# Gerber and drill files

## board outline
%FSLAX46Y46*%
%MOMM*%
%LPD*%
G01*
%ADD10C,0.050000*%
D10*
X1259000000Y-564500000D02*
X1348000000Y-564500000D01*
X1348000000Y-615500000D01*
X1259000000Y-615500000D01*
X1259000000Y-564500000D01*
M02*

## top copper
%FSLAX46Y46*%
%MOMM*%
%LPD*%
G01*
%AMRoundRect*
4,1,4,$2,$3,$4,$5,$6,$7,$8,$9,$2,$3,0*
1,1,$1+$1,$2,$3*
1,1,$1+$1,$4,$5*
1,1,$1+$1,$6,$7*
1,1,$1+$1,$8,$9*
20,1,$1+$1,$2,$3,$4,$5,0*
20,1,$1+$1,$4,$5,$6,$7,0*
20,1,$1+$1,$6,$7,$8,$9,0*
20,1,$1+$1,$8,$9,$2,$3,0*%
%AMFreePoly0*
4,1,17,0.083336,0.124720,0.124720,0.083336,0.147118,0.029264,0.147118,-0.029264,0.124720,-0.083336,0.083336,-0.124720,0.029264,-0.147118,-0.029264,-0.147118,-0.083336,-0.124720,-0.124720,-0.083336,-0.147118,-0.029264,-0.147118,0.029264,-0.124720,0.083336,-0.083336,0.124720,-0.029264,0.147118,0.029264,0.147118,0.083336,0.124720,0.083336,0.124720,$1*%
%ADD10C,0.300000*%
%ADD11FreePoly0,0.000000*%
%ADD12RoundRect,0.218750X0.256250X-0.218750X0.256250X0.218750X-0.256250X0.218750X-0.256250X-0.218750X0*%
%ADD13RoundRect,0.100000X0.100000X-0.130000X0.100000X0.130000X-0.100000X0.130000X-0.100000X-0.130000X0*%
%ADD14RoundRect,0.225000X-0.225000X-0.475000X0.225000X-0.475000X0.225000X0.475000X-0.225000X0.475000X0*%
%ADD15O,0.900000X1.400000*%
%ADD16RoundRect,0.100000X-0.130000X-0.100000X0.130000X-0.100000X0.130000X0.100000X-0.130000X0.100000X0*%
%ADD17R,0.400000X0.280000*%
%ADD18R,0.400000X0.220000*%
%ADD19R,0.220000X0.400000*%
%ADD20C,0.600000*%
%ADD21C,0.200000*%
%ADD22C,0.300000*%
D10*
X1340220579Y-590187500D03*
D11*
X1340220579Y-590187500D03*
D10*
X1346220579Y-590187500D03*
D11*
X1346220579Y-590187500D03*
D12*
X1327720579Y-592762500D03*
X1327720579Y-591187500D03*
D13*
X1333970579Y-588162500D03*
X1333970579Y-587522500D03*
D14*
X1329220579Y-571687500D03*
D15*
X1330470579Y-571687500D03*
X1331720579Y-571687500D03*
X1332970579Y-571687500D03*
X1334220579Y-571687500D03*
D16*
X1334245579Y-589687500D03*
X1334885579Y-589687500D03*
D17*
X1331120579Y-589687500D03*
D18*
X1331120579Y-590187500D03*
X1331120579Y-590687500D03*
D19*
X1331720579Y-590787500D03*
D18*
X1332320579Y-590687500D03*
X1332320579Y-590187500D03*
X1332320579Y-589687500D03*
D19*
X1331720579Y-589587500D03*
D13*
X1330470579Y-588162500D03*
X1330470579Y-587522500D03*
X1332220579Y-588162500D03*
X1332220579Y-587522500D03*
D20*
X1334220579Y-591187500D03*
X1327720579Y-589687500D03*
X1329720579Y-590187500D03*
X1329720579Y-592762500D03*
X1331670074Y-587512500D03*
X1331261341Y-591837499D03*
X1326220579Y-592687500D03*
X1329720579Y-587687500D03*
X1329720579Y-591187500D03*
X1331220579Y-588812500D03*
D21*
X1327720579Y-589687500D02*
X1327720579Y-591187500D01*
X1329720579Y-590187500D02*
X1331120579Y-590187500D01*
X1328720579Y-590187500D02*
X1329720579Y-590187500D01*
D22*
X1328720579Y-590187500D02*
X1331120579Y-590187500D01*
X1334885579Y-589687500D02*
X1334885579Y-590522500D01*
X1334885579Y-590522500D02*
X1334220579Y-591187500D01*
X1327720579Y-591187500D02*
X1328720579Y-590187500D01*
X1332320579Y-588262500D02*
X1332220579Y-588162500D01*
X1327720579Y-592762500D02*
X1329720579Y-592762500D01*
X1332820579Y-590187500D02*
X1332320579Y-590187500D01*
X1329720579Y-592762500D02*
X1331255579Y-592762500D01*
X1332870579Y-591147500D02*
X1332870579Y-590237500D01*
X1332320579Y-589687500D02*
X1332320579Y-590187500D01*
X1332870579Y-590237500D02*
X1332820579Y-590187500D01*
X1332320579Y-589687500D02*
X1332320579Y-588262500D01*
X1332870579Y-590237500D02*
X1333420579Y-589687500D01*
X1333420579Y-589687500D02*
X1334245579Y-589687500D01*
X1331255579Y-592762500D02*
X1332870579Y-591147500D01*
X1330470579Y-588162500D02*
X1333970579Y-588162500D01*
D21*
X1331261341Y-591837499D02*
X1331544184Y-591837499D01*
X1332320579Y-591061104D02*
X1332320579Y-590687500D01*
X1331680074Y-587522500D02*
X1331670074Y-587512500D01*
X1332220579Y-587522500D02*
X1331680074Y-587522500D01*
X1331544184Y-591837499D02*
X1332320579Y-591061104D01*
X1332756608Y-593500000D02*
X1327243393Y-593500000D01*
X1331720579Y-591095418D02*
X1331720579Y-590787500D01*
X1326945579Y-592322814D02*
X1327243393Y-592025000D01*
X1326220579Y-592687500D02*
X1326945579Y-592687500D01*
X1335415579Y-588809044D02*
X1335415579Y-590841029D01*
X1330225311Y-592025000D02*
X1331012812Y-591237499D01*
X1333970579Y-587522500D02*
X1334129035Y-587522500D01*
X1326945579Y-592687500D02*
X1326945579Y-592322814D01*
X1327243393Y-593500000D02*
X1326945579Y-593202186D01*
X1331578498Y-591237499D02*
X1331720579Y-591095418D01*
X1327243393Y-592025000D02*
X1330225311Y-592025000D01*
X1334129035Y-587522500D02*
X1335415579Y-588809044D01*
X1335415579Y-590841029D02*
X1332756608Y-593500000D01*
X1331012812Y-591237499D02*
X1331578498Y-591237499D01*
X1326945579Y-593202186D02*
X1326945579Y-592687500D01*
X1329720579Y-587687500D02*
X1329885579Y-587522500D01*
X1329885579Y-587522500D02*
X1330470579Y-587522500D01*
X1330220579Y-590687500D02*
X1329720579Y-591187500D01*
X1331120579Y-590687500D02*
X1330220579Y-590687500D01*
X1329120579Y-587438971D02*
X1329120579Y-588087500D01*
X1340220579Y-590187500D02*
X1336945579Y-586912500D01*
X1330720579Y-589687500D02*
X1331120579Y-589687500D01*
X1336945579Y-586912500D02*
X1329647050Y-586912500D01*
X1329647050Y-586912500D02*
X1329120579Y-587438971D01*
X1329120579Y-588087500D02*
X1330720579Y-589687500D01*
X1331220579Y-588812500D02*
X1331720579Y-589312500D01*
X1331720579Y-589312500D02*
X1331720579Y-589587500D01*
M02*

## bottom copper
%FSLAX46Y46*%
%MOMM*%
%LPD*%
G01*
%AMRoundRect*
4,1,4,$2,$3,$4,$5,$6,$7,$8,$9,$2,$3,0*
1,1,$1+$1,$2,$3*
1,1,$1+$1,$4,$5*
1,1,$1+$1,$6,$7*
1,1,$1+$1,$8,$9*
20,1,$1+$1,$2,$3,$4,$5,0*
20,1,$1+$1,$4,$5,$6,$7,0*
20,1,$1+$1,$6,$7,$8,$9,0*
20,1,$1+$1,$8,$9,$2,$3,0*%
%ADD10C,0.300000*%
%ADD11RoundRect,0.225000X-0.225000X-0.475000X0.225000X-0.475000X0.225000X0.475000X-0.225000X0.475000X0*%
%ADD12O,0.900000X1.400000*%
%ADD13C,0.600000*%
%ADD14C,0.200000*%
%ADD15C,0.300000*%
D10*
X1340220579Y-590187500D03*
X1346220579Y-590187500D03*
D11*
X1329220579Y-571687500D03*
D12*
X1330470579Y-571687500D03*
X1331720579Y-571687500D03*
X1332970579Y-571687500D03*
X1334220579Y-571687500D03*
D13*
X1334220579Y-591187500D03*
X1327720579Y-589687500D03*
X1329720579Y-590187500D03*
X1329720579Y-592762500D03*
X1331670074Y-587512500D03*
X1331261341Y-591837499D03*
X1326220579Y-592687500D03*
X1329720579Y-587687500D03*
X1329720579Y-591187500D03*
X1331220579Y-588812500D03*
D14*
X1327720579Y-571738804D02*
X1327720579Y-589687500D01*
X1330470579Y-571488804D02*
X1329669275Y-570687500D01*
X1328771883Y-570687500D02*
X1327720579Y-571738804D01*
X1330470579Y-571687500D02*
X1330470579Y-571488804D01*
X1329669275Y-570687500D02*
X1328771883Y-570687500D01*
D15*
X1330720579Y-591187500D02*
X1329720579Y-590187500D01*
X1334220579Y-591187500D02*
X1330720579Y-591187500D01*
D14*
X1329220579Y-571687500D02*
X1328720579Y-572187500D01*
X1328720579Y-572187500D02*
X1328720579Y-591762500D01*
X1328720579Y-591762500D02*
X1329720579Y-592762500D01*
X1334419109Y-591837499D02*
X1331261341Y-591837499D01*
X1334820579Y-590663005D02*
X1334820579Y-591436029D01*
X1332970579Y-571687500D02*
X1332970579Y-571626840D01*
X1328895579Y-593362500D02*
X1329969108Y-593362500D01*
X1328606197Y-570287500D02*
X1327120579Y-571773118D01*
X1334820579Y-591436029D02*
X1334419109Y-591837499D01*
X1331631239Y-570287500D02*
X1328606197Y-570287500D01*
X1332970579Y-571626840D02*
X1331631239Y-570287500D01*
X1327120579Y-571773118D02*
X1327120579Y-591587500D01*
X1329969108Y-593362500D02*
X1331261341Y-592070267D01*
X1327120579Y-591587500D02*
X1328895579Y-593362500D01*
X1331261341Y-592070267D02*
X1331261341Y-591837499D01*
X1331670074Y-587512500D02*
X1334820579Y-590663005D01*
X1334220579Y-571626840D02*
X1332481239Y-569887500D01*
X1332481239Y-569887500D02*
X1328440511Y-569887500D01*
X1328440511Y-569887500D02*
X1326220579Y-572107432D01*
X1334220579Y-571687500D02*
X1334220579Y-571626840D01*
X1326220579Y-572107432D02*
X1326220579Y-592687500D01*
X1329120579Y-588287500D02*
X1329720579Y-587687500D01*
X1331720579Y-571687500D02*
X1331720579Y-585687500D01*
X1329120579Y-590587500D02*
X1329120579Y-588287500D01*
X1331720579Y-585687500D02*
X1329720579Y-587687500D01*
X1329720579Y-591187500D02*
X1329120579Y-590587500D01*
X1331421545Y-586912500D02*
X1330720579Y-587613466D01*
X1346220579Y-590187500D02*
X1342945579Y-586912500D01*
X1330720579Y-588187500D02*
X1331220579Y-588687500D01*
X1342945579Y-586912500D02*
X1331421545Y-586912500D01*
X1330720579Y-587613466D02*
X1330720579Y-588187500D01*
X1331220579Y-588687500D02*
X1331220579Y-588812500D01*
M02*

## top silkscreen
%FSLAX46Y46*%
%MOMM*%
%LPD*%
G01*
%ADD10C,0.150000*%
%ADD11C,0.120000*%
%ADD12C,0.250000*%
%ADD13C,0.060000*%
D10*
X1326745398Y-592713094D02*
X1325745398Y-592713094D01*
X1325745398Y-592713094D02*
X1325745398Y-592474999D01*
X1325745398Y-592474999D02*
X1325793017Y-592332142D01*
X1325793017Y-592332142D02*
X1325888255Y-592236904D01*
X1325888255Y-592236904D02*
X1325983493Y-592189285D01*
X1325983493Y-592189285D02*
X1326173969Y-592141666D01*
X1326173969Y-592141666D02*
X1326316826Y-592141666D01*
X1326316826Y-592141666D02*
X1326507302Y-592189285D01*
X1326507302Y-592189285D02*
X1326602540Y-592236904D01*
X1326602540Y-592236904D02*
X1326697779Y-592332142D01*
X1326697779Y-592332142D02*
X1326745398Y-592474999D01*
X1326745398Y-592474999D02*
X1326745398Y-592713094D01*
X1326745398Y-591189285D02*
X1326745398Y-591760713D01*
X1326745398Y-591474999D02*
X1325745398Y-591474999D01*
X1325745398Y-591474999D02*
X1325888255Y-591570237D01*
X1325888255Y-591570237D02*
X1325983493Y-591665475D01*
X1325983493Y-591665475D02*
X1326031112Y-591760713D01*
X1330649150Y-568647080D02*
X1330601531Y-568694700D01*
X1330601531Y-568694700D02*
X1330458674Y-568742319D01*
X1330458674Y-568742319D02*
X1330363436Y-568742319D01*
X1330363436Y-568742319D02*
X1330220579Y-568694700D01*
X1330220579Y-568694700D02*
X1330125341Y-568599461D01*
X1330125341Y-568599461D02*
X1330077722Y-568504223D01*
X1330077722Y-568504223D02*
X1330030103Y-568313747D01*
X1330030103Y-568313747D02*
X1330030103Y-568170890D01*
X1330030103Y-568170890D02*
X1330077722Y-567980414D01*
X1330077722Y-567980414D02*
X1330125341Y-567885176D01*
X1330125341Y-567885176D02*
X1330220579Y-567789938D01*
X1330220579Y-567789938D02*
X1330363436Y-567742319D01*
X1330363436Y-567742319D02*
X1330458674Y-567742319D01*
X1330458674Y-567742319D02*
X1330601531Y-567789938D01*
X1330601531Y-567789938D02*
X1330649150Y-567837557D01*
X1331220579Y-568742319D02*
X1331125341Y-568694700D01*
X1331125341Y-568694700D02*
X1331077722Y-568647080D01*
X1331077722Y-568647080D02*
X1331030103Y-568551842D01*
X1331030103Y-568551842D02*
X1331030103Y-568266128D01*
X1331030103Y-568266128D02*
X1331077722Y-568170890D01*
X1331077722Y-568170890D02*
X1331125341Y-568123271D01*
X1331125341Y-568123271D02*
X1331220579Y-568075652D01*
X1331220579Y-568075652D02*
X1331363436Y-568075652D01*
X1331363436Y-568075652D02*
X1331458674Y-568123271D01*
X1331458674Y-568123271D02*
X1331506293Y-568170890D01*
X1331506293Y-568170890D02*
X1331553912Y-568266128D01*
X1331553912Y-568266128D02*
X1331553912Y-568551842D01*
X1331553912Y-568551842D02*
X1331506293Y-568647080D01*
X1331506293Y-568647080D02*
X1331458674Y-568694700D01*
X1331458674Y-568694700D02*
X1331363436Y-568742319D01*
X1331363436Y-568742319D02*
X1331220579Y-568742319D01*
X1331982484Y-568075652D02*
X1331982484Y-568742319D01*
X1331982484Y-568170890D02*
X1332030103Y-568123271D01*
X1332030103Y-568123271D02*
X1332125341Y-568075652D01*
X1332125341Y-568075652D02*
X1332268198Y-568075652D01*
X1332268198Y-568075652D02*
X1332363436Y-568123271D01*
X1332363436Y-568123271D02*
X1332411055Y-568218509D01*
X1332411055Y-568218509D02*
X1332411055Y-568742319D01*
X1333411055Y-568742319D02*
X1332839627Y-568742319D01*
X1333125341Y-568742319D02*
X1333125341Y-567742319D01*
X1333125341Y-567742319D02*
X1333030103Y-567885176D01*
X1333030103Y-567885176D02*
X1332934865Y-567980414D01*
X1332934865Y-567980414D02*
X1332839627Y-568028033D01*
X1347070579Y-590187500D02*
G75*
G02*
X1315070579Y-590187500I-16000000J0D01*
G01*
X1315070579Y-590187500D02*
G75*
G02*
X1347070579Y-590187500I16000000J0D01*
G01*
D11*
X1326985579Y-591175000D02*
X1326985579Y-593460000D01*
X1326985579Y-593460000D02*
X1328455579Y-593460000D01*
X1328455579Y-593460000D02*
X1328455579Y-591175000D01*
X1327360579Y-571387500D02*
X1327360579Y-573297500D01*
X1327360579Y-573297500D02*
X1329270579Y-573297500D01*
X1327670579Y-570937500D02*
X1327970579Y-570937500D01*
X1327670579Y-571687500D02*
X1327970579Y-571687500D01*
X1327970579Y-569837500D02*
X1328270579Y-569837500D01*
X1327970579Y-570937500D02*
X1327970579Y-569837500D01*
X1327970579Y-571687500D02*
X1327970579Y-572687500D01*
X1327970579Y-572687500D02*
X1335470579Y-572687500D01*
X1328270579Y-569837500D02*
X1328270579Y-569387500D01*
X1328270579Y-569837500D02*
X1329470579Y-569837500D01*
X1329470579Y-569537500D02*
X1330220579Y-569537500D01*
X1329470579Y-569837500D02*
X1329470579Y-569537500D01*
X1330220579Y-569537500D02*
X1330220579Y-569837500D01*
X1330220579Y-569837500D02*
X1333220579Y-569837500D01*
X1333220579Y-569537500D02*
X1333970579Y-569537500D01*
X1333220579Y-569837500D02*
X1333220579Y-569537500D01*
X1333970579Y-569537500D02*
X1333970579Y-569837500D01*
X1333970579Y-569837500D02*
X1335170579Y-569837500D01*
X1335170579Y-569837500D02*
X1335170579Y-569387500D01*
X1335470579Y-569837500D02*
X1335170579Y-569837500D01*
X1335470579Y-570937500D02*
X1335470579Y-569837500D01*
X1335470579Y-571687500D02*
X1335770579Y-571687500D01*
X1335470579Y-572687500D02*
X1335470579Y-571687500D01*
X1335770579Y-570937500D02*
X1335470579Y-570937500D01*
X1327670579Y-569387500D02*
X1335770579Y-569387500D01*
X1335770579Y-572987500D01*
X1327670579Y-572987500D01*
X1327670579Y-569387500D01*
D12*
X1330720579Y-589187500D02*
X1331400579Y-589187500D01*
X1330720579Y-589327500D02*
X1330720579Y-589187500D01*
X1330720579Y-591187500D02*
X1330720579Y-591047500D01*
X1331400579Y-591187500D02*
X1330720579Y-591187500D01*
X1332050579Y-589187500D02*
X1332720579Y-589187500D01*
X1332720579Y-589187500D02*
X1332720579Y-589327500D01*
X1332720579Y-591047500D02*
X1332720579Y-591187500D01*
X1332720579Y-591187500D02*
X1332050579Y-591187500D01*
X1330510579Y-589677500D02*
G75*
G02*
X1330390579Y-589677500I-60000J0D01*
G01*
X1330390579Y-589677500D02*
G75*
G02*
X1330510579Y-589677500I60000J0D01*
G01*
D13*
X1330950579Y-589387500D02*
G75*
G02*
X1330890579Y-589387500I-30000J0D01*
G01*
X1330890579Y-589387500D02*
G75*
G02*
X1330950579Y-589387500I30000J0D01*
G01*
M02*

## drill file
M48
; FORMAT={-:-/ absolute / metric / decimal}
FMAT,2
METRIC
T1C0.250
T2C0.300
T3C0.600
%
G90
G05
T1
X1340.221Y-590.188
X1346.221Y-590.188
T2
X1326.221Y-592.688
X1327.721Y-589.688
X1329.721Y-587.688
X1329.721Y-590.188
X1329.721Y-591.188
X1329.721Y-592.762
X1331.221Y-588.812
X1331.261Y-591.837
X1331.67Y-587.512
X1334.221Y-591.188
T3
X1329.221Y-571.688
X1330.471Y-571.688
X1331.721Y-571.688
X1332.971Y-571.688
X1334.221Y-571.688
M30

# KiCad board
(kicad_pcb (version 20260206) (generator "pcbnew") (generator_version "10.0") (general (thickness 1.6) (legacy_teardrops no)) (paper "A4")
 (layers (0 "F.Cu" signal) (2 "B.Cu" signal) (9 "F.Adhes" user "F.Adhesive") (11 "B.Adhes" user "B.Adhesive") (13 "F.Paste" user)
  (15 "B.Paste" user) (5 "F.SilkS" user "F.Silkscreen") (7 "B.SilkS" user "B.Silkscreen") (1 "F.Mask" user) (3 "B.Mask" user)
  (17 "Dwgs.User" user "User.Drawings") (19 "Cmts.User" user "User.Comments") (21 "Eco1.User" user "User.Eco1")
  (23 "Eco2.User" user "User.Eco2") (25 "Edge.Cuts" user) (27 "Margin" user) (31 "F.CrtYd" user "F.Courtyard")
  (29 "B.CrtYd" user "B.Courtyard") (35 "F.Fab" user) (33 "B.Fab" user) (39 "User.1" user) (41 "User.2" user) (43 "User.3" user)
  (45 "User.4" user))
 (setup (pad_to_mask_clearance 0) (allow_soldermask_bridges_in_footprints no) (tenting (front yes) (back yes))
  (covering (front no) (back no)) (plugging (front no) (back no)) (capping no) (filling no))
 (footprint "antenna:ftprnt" (layer "F.Cu") (at 1331.070579 575.1875)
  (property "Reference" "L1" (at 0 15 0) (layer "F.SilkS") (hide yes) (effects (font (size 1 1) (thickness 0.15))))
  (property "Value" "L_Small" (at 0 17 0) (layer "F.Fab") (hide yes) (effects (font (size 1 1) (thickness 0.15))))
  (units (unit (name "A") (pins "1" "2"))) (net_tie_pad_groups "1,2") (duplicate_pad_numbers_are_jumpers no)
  (fp_circle (center 0 15) (end 0 31) (stroke (width 0.15) (type solid)) (fill no) (layer "F.SilkS"))
  (pad "1" thru_hole circle (at 9.15 15) (size 0.3 0.3) (drill 0.25) (layers "*.Cu" "*.Mask") (remove_unused_layers no) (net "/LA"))
  (pad "1" smd custom (at 9.15 15) (size 0.3 0.3) (layers "F.Cu") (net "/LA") (zone_connect 0) (thermal_bridge_angle 90)
   (options (clearance outline) (anchor circle)) (primitives))
  (pad "2" thru_hole circle (at 15.15 15) (size 0.3 0.3) (drill 0.25) (layers "*.Cu" "*.Mask") (remove_unused_layers no) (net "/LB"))
  (pad "2" smd custom (at 15.15 15) (size 0.3 0.3) (layers "F.Cu") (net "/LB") (zone_connect 0) (thermal_bridge_angle 90)
   (options (clearance outline) (anchor circle)) (primitives)))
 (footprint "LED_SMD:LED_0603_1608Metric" (layer "F.Cu") (at 1327.720579 591.975 90)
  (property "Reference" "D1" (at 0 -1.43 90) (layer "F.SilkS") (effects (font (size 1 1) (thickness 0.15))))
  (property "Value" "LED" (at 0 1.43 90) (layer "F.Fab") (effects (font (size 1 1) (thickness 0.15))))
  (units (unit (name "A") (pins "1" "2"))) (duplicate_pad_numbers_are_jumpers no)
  (fp_line (start 0.8 -0.735) (end -1.485 -0.735) (stroke (width 0.12) (type solid)) (layer "F.SilkS"))
  (fp_line (start -1.485 -0.735) (end -1.485 0.735) (stroke (width 0.12) (type solid)) (layer "F.SilkS"))
  (fp_line (start -1.485 0.735) (end 0.8 0.735) (stroke (width 0.12) (type solid)) (layer "F.SilkS"))
  (pad "1" smd roundrect (at -0.7875 0 90) (size 0.875 0.95) (layers "F.Cu" "F.Mask" "F.Paste") (roundrect_rratio 0.25) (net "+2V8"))
  (pad "2" smd roundrect (at 0.7875 0 90) (size 0.875 0.95) (layers "F.Cu" "F.Mask" "F.Paste") (roundrect_rratio 0.25) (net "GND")))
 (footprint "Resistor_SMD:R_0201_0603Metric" (layer "F.Cu") (at 1333.970579 587.8425 90)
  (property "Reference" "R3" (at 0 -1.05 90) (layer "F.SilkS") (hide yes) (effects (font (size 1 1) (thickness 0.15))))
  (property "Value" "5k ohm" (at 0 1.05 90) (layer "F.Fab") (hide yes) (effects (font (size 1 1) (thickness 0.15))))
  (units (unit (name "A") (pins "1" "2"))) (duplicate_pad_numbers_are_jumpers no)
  (pad "" smd roundrect (at -0.345 0 90) (size 0.318 0.36) (layers "F.Paste") (roundrect_rratio 0.25))
  (pad "" smd roundrect (at 0.345 0 90) (size 0.318 0.36) (layers "F.Paste") (roundrect_rratio 0.25))
  (pad "1" smd roundrect (at -0.32 0 90) (size 0.46 0.4) (layers "F.Cu" "F.Mask") (roundrect_rratio 0.25) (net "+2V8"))
  (pad "2" smd roundrect (at 0.32 0 90) (size 0.46 0.4) (layers "F.Cu" "F.Mask") (roundrect_rratio 0.25) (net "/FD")))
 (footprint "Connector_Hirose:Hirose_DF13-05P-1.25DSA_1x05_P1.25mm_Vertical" (layer "F.Cu") (at 1329.220579 571.6875)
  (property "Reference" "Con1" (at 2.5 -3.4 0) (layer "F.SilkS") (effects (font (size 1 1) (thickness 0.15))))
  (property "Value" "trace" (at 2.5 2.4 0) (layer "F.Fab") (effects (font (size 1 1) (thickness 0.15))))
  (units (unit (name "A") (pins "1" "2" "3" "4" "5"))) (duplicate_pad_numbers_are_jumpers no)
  (fp_line (start -1.86 -0.3) (end -1.86 1.61) (stroke (width 0.12) (type solid)) (layer "F.SilkS"))
  (fp_line (start -1.86 1.61) (end 0.05 1.61) (stroke (width 0.12) (type solid)) (layer "F.SilkS"))
  (fp_line (start -1.55 -0.75) (end -1.25 -0.75) (stroke (width 0.12) (type solid)) (layer "F.SilkS"))
  (fp_line (start -1.55 0) (end -1.25 0) (stroke (width 0.12) (type solid)) (layer "F.SilkS"))
  (fp_line (start -1.25 -1.85) (end -0.95 -1.85) (stroke (width 0.12) (type solid)) (layer "F.SilkS"))
  (fp_line (start -1.25 -0.75) (end -1.25 -1.85) (stroke (width 0.12) (type solid)) (layer "F.SilkS"))
  (fp_line (start -1.25 0) (end -1.25 1) (stroke (width 0.12) (type solid)) (layer "F.SilkS"))
  (fp_line (start -1.25 1) (end 6.25 1) (stroke (width 0.12) (type solid)) (layer "F.SilkS"))
  (fp_line (start -0.95 -1.85) (end -0.95 -2.3) (stroke (width 0.12) (type solid)) (layer "F.SilkS"))
  (fp_line (start -0.95 -1.85) (end 0.25 -1.85) (stroke (width 0.12) (type solid)) (layer "F.SilkS"))
  (fp_line (start 0.25 -2.15) (end 1 -2.15) (stroke (width 0.12) (type solid)) (layer "F.SilkS"))
  (fp_line (start 0.25 -1.85) (end 0.25 -2.15) (stroke (width 0.12) (type solid)) (layer "F.SilkS"))
  (fp_line (start 1 -2.15) (end 1 -1.85) (stroke (width 0.12) (type solid)) (layer "F.SilkS"))
  (fp_line (start 1 -1.85) (end 4 -1.85) (stroke (width 0.12) (type solid)) (layer "F.SilkS"))
  (fp_line (start 4 -2.15) (end 4.75 -2.15) (stroke (width 0.12) (type solid)) (layer "F.SilkS"))
  (fp_line (start 4 -1.85) (end 4 -2.15) (stroke (width 0.12) (type solid)) (layer "F.SilkS"))
  (fp_line (start 4.75 -2.15) (end 4.75 -1.85) (stroke (width 0.12) (type solid)) (layer "F.SilkS"))
  (fp_line (start 4.75 -1.85) (end 5.95 -1.85) (stroke (width 0.12) (type solid)) (layer "F.SilkS"))
  (fp_line (start 5.95 -1.85) (end 5.95 -2.3) (stroke (width 0.12) (type solid)) (layer "F.SilkS"))
  (fp_line (start 6.25 -1.85) (end 5.95 -1.85) (stroke (width 0.12) (type solid)) (layer "F.SilkS"))
  (fp_line (start 6.25 -0.75) (end 6.25 -1.85) (stroke (width 0.12) (type solid)) (layer "F.SilkS"))
  (fp_line (start 6.25 0) (end 6.55 0) (stroke (width 0.12) (type solid)) (layer "F.SilkS"))
  (fp_line (start 6.25 1) (end 6.25 0) (stroke (width 0.12) (type solid)) (layer "F.SilkS"))
  (fp_line (start 6.55 -0.75) (end 6.25 -0.75) (stroke (width 0.12) (type solid)) (layer "F.SilkS"))
  (fp_rect (start -1.55 -2.3) (end 6.55 1.3) (stroke (width 0.12) (type solid)) (fill no) (layer "F.SilkS"))
  (pad "1" thru_hole roundrect (at 0 0) (size 0.9 1.4) (drill 0.6) (layers "*.Cu" "*.Mask") (remove_unused_layers no)
   (roundrect_rratio 0.25) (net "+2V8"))
  (pad "2" thru_hole oval (at 1.25 0) (size 0.9 1.4) (drill 0.6) (layers "*.Cu" "*.Mask") (remove_unused_layers no) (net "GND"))
  (pad "3" thru_hole oval (at 2.5 0) (size 0.9 1.4) (drill 0.6) (layers "*.Cu" "*.Mask") (remove_unused_layers no) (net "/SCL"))
  (pad "4" thru_hole oval (at 3.75 0) (size 0.9 1.4) (drill 0.6) (layers "*.Cu" "*.Mask") (remove_unused_layers no) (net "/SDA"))
  (pad "5" thru_hole oval (at 5 0) (size 0.9 1.4) (drill 0.6) (layers "*.Cu" "*.Mask") (remove_unused_layers no) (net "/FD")))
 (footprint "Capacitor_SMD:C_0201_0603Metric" (layer "F.Cu") (at 1334.565579 589.6875)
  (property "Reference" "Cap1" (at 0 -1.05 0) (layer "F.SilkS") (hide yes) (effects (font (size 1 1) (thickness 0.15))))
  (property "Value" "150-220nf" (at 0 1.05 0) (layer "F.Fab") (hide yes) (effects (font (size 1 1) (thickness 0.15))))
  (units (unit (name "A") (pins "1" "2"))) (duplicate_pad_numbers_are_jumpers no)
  (pad "" smd roundrect (at -0.345 0) (size 0.318 0.36) (layers "F.Paste") (roundrect_rratio 0.25))
  (pad "" smd roundrect (at 0.345 0) (size 0.318 0.36) (layers "F.Paste") (roundrect_rratio 0.25))
  (pad "1" smd roundrect (at -0.32 0) (size 0.46 0.4) (layers "F.Cu" "F.Mask") (roundrect_rratio 0.25) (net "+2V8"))
  (pad "2" smd roundrect (at 0.32 0) (size 0.46 0.4) (layers "F.Cu" "F.Mask") (roundrect_rratio 0.25) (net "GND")))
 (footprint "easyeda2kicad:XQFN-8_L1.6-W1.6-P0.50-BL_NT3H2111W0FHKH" (layer "F.Cu") (at 1331.720579 590.1875)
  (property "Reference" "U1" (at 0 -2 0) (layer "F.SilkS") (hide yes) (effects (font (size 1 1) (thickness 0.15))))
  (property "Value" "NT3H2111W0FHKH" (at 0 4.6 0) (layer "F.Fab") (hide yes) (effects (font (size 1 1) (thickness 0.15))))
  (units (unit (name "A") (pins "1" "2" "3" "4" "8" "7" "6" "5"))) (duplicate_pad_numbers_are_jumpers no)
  (fp_line (start -1 -1) (end -0.32 -1) (stroke (width 0.25) (type solid)) (layer "F.SilkS"))
  (fp_line (start -1 -0.86) (end -1 -1) (stroke (width 0.25) (type solid)) (layer "F.SilkS"))
  (fp_line (start -1 1) (end -1 0.86) (stroke (width 0.25) (type solid)) (layer "F.SilkS"))
  (fp_line (start -0.32 1) (end -1 1) (stroke (width 0.25) (type solid)) (layer "F.SilkS"))
  (fp_line (start 0.33 -1) (end 1 -1) (stroke (width 0.25) (type solid)) (layer "F.SilkS"))
  (fp_line (start 1 -1) (end 1 -0.86) (stroke (width 0.25) (type solid)) (layer "F.SilkS"))
  (fp_line (start 1 0.86) (end 1 1) (stroke (width 0.25) (type solid)) (layer "F.SilkS"))
  (fp_line (start 1 1) (end 0.33 1) (stroke (width 0.25) (type solid)) (layer "F.SilkS"))
  (fp_circle (center -1.27 -0.51) (end -1.21 -0.51) (stroke (width 0.25) (type solid)) (fill no) (layer "F.SilkS"))
  (fp_circle (center -0.8 -0.8) (end -0.77 -0.8) (stroke (width 0.06) (type solid)) (fill no) (layer "F.SilkS"))
  (pad "1" smd rect (at -0.6 -0.5) (size 0.4 0.28) (layers "F.Cu" "F.Mask" "F.Paste") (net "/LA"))
  (pad "2" smd rect (at -0.6 0) (size 0.4 0.22) (layers "F.Cu" "F.Mask" "F.Paste") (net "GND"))
  (pad "3" smd rect (at -0.6 0.5) (size 0.4 0.22) (layers "F.Cu" "F.Mask" "F.Paste") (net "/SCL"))
  (pad "4" smd rect (at 0 0.6 90) (size 0.4 0.22) (layers "F.Cu" "F.Mask" "F.Paste") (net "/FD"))
  (pad "5" smd rect (at 0.6 0.5) (size 0.4 0.22) (layers "F.Cu" "F.Mask" "F.Paste") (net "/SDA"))
  (pad "6" smd rect (at 0.6 0) (size 0.4 0.22) (layers "F.Cu" "F.Mask" "F.Paste") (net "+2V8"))
  (pad "7" smd rect (at 0.6 -0.5) (size 0.4 0.22) (layers "F.Cu" "F.Mask" "F.Paste") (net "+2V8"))
  (pad "8" smd rect (at 0 -0.6 90) (size 0.4 0.22) (layers "F.Cu" "F.Mask" "F.Paste") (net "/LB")))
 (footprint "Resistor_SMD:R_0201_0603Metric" (layer "F.Cu") (at 1330.470579 587.8425 90)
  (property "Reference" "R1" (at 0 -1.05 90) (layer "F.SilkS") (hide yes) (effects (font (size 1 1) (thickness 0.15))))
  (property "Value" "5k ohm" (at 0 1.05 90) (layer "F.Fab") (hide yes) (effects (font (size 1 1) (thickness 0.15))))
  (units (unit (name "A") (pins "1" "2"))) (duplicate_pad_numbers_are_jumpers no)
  (pad "" smd roundrect (at -0.345 0 90) (size 0.318 0.36) (layers "F.Paste") (roundrect_rratio 0.25))
  (pad "" smd roundrect (at 0.345 0 90) (size 0.318 0.36) (layers "F.Paste") (roundrect_rratio 0.25))
  (pad "1" smd roundrect (at -0.32 0 90) (size 0.46 0.4) (layers "F.Cu" "F.Mask") (roundrect_rratio 0.25) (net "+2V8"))
  (pad "2" smd roundrect (at 0.32 0 90) (size 0.46 0.4) (layers "F.Cu" "F.Mask") (roundrect_rratio 0.25) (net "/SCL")))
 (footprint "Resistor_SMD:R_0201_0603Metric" (layer "F.Cu") (at 1332.220579 587.8425 90)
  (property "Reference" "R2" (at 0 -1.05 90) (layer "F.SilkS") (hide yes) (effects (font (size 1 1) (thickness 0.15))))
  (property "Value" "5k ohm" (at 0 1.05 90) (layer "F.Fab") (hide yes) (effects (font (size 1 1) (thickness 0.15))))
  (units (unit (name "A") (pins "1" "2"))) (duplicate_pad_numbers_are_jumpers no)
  (pad "" smd roundrect (at -0.345 0 90) (size 0.318 0.36) (layers "F.Paste") (roundrect_rratio 0.25))
  (pad "" smd roundrect (at 0.345 0 90) (size 0.318 0.36) (layers "F.Paste") (roundrect_rratio 0.25))
  (pad "1" smd roundrect (at -0.32 0 90) (size 0.46 0.4) (layers "F.Cu" "F.Mask") (roundrect_rratio 0.25) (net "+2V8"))
  (pad "2" smd roundrect (at 0.32 0 90) (size 0.46 0.4) (layers "F.Cu" "F.Mask") (roundrect_rratio 0.25) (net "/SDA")))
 (gr_rect (start 1259 564.5) (end 1348 615.5) (stroke (width 0.05) (type default)) (fill no) (layer "Edge.Cuts"))
 (segment (start 1327.720579 589.6875) (end 1327.720579 591.1875) (width 0.2) (layer "F.Cu") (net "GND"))
 (segment (start 1329.720579 590.1875) (end 1331.120579 590.1875) (width 0.2) (layer "F.Cu") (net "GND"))
 (segment (start 1328.720579 590.1875) (end 1329.720579 590.1875) (width 0.2) (layer "F.Cu") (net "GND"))
 (segment (start 1328.720579 590.1875) (end 1331.120579 590.1875) (width 0.3) (layer "F.Cu") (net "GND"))
 (segment (start 1334.885579 589.6875) (end 1334.885579 590.5225) (width 0.3) (layer "F.Cu") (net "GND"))
 (segment (start 1334.885579 590.5225) (end 1334.220579 591.1875) (width 0.3) (layer "F.Cu") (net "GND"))
 (segment (start 1327.720579 591.1875) (end 1328.720579 590.1875) (width 0.3) (layer "F.Cu") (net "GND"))
 (via (at 1334.220579 591.1875) (size 0.6) (drill 0.3) (layers "F.Cu" "B.Cu") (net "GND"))
 (via (at 1327.720579 589.6875) (size 0.6) (drill 0.3) (layers "F.Cu" "B.Cu") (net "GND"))
 (via (at 1329.720579 590.1875) (size 0.6) (drill 0.3) (layers "F.Cu" "B.Cu") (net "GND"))
 (segment (start 1327.720579 571.738804) (end 1327.720579 589.6875) (width 0.2) (layer "B.Cu") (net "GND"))
 (segment (start 1330.470579 571.488804) (end 1329.669275 570.6875) (width 0.2) (layer "B.Cu") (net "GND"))
 (segment (start 1328.771883 570.6875) (end 1327.720579 571.738804) (width 0.2) (layer "B.Cu") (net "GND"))
 (segment (start 1330.470579 571.6875) (end 1330.470579 571.488804) (width 0.2) (layer "B.Cu") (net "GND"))
 (segment (start 1329.669275 570.6875) (end 1328.771883 570.6875) (width 0.2) (layer "B.Cu") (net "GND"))
 (segment (start 1330.720579 591.1875) (end 1329.720579 590.1875) (width 0.3) (layer "B.Cu") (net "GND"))
 (segment (start 1334.220579 591.1875) (end 1330.720579 591.1875) (width 0.3) (layer "B.Cu") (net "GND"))
 (segment (start 1332.320579 588.2625) (end 1332.220579 588.1625) (width 0.3) (layer "F.Cu") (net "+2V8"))
 (segment (start 1327.720579 592.7625) (end 1329.720579 592.7625) (width 0.3) (layer "F.Cu") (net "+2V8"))
 (segment (start 1332.820579 590.1875) (end 1332.320579 590.1875) (width 0.3) (layer "F.Cu") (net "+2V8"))
 (segment (start 1329.720579 592.7625) (end 1331.255579 592.7625) (width 0.3) (layer "F.Cu") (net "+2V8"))
 (segment (start 1332.870579 591.1475) (end 1332.870579 590.2375) (width 0.3) (layer "F.Cu") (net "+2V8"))
 (segment (start 1332.320579 589.6875) (end 1332.320579 590.1875) (width 0.3) (layer "F.Cu") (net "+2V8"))
 (segment (start 1332.870579 590.2375) (end 1332.820579 590.1875) (width 0.3) (layer "F.Cu") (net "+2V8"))
 (segment (start 1332.320579 589.6875) (end 1332.320579 588.2625) (width 0.3) (layer "F.Cu") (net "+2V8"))
 (segment (start 1332.870579 590.2375) (end 1333.420579 589.6875) (width 0.3) (layer "F.Cu") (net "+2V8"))
 (segment (start 1333.420579 589.6875) (end 1334.245579 589.6875) (width 0.3) (layer "F.Cu") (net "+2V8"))
 (segment (start 1331.255579 592.7625) (end 1332.870579 591.1475) (width 0.3) (layer "F.Cu") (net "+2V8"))
 (segment (start 1330.470579 588.1625) (end 1333.970579 588.1625) (width 0.3) (layer "F.Cu") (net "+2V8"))
 (via (at 1329.720579 592.7625) (size 0.6) (drill 0.3) (layers "F.Cu" "B.Cu") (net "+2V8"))
 (segment (start 1329.220579 571.6875) (end 1328.720579 572.1875) (width 0.2) (layer "B.Cu") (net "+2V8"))
 (segment (start 1328.720579 572.1875) (end 1328.720579 591.7625) (width 0.2) (layer "B.Cu") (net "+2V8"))
 (segment (start 1328.720579 591.7625) (end 1329.720579 592.7625) (width 0.2) (layer "B.Cu") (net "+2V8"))
 (segment (start 1331.261341 591.837499) (end 1331.544184 591.837499) (width 0.2) (layer "F.Cu") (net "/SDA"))
 (segment (start 1332.320579 591.061104) (end 1332.320579 590.6875) (width 0.2) (layer "F.Cu") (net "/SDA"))
 (segment (start 1331.680074 587.5225) (end 1331.670074 587.5125) (width 0.2) (layer "F.Cu") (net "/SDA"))
 (segment (start 1332.220579 587.5225) (end 1331.680074 587.5225) (width 0.2) (layer "F.Cu") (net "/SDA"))
 (segment (start 1331.544184 591.837499) (end 1332.320579 591.061104) (width 0.2) (layer "F.Cu") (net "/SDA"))
 (via (at 1331.670074 587.5125) (size 0.6) (drill 0.3) (layers "F.Cu" "B.Cu") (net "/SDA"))
 (via (at 1331.261341 591.837499) (size 0.6) (drill 0.3) (layers "F.Cu" "B.Cu") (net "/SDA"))
 (segment (start 1334.419109 591.837499) (end 1331.261341 591.837499) (width 0.2) (layer "B.Cu") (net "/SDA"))
 (segment (start 1334.820579 590.663005) (end 1334.820579 591.436029) (width 0.2) (layer "B.Cu") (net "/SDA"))
 (segment (start 1332.970579 571.6875) (end 1332.970579 571.62684) (width 0.2) (layer "B.Cu") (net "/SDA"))
 (segment (start 1328.895579 593.3625) (end 1329.969108 593.3625) (width 0.2) (layer "B.Cu") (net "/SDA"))
 (segment (start 1328.606197 570.2875) (end 1327.120579 571.773118) (width 0.2) (layer "B.Cu") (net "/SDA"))
 (segment (start 1334.820579 591.436029) (end 1334.419109 591.837499) (width 0.2) (layer "B.Cu") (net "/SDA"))
 (segment (start 1331.631239 570.2875) (end 1328.606197 570.2875) (width 0.2) (layer "B.Cu") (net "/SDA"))
 (segment (start 1332.970579 571.62684) (end 1331.631239 570.2875) (width 0.2) (layer "B.Cu") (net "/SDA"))
 (segment (start 1327.120579 571.773118) (end 1327.120579 591.5875) (width 0.2) (layer "B.Cu") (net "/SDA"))
 (segment (start 1329.969108 593.3625) (end 1331.261341 592.070267) (width 0.2) (layer "B.Cu") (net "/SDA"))
 (segment (start 1327.120579 591.5875) (end 1328.895579 593.3625) (width 0.2) (layer "B.Cu") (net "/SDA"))
 (segment (start 1331.261341 592.070267) (end 1331.261341 591.837499) (width 0.2) (layer "B.Cu") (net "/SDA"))
 (segment (start 1331.670074 587.5125) (end 1334.820579 590.663005) (width 0.2) (layer "B.Cu") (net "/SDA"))
 (segment (start 1332.756608 593.5) (end 1327.243393 593.5) (width 0.2) (layer "F.Cu") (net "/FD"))
 (segment (start 1331.720579 591.095418) (end 1331.720579 590.7875) (width 0.2) (layer "F.Cu") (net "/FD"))
 (segment (start 1326.945579 592.322814) (end 1327.243393 592.025) (width 0.2) (layer "F.Cu") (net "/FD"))
 (segment (start 1326.220579 592.6875) (end 1326.945579 592.6875) (width 0.2) (layer "F.Cu") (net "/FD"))
 (segment (start 1335.415579 588.809044) (end 1335.415579 590.841029) (width 0.2) (layer "F.Cu") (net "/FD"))
 (segment (start 1330.225311 592.025) (end 1331.012812 591.237499) (width 0.2) (layer "F.Cu") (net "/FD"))
 (segment (start 1333.970579 587.5225) (end 1334.129035 587.5225) (width 0.2) (layer "F.Cu") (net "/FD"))
 (segment (start 1326.945579 592.6875) (end 1326.945579 592.322814) (width 0.2) (layer "F.Cu") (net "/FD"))
 (segment (start 1327.243393 593.5) (end 1326.945579 593.202186) (width 0.2) (layer "F.Cu") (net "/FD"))
 (segment (start 1331.578498 591.237499) (end 1331.720579 591.095418) (width 0.2) (layer "F.Cu") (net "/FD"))
 (segment (start 1327.243393 592.025) (end 1330.225311 592.025) (width 0.2) (layer "F.Cu") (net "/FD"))
 (segment (start 1334.129035 587.5225) (end 1335.415579 588.809044) (width 0.2) (layer "F.Cu") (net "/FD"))
 (segment (start 1335.415579 590.841029) (end 1332.756608 593.5) (width 0.2) (layer "F.Cu") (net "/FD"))
 (segment (start 1331.012812 591.237499) (end 1331.578498 591.237499) (width 0.2) (layer "F.Cu") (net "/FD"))
 (segment (start 1326.945579 593.202186) (end 1326.945579 592.6875) (width 0.2) (layer "F.Cu") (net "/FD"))
 (via (at 1326.220579 592.6875) (size 0.6) (drill 0.3) (layers "F.Cu" "B.Cu") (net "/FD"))
 (segment (start 1334.220579 571.62684) (end 1332.481239 569.8875) (width 0.2) (layer "B.Cu") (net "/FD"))
 (segment (start 1332.481239 569.8875) (end 1328.440511 569.8875) (width 0.2) (layer "B.Cu") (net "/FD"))
 (segment (start 1328.440511 569.8875) (end 1326.220579 572.107432) (width 0.2) (layer "B.Cu") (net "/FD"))
 (segment (start 1334.220579 571.6875) (end 1334.220579 571.62684) (width 0.2) (layer "B.Cu") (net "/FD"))
 (segment (start 1326.220579 572.107432) (end 1326.220579 592.6875) (width 0.2) (layer "B.Cu") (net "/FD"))
 (segment (start 1329.720579 587.6875) (end 1329.885579 587.5225) (width 0.2) (layer "F.Cu") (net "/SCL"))
 (segment (start 1329.885579 587.5225) (end 1330.470579 587.5225) (width 0.2) (layer "F.Cu") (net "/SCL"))
 (segment (start 1330.220579 590.6875) (end 1329.720579 591.1875) (width 0.2) (layer "F.Cu") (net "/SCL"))
 (segment (start 1331.120579 590.6875) (end 1330.220579 590.6875) (width 0.2) (layer "F.Cu") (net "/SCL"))
 (via (at 1329.720579 587.6875) (size 0.6) (drill 0.3) (layers "F.Cu" "B.Cu") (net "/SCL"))
 (via (at 1329.720579 591.1875) (size 0.6) (drill 0.3) (layers "F.Cu" "B.Cu") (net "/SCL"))
 (segment (start 1329.120579 588.2875) (end 1329.720579 587.6875) (width 0.2) (layer "B.Cu") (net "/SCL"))
 (segment (start 1331.720579 571.6875) (end 1331.720579 585.6875) (width 0.2) (layer "B.Cu") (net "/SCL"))
 (segment (start 1329.120579 590.5875) (end 1329.120579 588.2875) (width 0.2) (layer "B.Cu") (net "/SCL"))
 (segment (start 1331.720579 585.6875) (end 1329.720579 587.6875) (width 0.2) (layer "B.Cu") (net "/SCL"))
 (segment (start 1329.720579 591.1875) (end 1329.120579 590.5875) (width 0.2) (layer "B.Cu") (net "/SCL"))
 (segment (start 1329.120579 587.438971) (end 1329.120579 588.0875) (width 0.2) (layer "F.Cu") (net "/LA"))
 (segment (start 1340.220579 590.1875) (end 1336.945579 586.9125) (width 0.2) (layer "F.Cu") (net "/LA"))
 (segment (start 1330.720579 589.6875) (end 1331.120579 589.6875) (width 0.2) (layer "F.Cu") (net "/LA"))
 (segment (start 1336.945579 586.9125) (end 1329.64705 586.9125) (width 0.2) (layer "F.Cu") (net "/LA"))
 (segment (start 1329.64705 586.9125) (end 1329.120579 587.438971) (width 0.2) (layer "F.Cu") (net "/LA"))
 (segment (start 1329.120579 588.0875) (end 1330.720579 589.6875) (width 0.2) (layer "F.Cu") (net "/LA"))
 (segment (start 1331.220579 588.8125) (end 1331.720579 589.3125) (width 0.2) (layer "F.Cu") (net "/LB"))
 (segment (start 1331.720579 589.3125) (end 1331.720579 589.5875) (width 0.2) (layer "F.Cu") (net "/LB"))
 (via (at 1331.220579 588.8125) (size 0.6) (drill 0.3) (layers "F.Cu" "B.Cu") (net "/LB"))
 (segment (start 1331.421545 586.9125) (end 1330.720579 587.613466) (width 0.2) (layer "B.Cu") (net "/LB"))
 (segment (start 1346.220579 590.1875) (end 1342.945579 586.9125) (width 0.2) (layer "B.Cu") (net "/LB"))
 (segment (start 1330.720579 588.1875) (end 1331.220579 588.6875) (width 0.2) (layer "B.Cu") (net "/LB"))
 (segment (start 1342.945579 586.9125) (end 1331.421545 586.9125) (width 0.2) (layer "B.Cu") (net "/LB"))
 (segment (start 1330.720579 587.613466) (end 1330.720579 588.1875) (width 0.2) (layer "B.Cu") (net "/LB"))
 (segment (start 1331.220579 588.6875) (end 1331.220579 588.8125) (width 0.2) (layer "B.Cu") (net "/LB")))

